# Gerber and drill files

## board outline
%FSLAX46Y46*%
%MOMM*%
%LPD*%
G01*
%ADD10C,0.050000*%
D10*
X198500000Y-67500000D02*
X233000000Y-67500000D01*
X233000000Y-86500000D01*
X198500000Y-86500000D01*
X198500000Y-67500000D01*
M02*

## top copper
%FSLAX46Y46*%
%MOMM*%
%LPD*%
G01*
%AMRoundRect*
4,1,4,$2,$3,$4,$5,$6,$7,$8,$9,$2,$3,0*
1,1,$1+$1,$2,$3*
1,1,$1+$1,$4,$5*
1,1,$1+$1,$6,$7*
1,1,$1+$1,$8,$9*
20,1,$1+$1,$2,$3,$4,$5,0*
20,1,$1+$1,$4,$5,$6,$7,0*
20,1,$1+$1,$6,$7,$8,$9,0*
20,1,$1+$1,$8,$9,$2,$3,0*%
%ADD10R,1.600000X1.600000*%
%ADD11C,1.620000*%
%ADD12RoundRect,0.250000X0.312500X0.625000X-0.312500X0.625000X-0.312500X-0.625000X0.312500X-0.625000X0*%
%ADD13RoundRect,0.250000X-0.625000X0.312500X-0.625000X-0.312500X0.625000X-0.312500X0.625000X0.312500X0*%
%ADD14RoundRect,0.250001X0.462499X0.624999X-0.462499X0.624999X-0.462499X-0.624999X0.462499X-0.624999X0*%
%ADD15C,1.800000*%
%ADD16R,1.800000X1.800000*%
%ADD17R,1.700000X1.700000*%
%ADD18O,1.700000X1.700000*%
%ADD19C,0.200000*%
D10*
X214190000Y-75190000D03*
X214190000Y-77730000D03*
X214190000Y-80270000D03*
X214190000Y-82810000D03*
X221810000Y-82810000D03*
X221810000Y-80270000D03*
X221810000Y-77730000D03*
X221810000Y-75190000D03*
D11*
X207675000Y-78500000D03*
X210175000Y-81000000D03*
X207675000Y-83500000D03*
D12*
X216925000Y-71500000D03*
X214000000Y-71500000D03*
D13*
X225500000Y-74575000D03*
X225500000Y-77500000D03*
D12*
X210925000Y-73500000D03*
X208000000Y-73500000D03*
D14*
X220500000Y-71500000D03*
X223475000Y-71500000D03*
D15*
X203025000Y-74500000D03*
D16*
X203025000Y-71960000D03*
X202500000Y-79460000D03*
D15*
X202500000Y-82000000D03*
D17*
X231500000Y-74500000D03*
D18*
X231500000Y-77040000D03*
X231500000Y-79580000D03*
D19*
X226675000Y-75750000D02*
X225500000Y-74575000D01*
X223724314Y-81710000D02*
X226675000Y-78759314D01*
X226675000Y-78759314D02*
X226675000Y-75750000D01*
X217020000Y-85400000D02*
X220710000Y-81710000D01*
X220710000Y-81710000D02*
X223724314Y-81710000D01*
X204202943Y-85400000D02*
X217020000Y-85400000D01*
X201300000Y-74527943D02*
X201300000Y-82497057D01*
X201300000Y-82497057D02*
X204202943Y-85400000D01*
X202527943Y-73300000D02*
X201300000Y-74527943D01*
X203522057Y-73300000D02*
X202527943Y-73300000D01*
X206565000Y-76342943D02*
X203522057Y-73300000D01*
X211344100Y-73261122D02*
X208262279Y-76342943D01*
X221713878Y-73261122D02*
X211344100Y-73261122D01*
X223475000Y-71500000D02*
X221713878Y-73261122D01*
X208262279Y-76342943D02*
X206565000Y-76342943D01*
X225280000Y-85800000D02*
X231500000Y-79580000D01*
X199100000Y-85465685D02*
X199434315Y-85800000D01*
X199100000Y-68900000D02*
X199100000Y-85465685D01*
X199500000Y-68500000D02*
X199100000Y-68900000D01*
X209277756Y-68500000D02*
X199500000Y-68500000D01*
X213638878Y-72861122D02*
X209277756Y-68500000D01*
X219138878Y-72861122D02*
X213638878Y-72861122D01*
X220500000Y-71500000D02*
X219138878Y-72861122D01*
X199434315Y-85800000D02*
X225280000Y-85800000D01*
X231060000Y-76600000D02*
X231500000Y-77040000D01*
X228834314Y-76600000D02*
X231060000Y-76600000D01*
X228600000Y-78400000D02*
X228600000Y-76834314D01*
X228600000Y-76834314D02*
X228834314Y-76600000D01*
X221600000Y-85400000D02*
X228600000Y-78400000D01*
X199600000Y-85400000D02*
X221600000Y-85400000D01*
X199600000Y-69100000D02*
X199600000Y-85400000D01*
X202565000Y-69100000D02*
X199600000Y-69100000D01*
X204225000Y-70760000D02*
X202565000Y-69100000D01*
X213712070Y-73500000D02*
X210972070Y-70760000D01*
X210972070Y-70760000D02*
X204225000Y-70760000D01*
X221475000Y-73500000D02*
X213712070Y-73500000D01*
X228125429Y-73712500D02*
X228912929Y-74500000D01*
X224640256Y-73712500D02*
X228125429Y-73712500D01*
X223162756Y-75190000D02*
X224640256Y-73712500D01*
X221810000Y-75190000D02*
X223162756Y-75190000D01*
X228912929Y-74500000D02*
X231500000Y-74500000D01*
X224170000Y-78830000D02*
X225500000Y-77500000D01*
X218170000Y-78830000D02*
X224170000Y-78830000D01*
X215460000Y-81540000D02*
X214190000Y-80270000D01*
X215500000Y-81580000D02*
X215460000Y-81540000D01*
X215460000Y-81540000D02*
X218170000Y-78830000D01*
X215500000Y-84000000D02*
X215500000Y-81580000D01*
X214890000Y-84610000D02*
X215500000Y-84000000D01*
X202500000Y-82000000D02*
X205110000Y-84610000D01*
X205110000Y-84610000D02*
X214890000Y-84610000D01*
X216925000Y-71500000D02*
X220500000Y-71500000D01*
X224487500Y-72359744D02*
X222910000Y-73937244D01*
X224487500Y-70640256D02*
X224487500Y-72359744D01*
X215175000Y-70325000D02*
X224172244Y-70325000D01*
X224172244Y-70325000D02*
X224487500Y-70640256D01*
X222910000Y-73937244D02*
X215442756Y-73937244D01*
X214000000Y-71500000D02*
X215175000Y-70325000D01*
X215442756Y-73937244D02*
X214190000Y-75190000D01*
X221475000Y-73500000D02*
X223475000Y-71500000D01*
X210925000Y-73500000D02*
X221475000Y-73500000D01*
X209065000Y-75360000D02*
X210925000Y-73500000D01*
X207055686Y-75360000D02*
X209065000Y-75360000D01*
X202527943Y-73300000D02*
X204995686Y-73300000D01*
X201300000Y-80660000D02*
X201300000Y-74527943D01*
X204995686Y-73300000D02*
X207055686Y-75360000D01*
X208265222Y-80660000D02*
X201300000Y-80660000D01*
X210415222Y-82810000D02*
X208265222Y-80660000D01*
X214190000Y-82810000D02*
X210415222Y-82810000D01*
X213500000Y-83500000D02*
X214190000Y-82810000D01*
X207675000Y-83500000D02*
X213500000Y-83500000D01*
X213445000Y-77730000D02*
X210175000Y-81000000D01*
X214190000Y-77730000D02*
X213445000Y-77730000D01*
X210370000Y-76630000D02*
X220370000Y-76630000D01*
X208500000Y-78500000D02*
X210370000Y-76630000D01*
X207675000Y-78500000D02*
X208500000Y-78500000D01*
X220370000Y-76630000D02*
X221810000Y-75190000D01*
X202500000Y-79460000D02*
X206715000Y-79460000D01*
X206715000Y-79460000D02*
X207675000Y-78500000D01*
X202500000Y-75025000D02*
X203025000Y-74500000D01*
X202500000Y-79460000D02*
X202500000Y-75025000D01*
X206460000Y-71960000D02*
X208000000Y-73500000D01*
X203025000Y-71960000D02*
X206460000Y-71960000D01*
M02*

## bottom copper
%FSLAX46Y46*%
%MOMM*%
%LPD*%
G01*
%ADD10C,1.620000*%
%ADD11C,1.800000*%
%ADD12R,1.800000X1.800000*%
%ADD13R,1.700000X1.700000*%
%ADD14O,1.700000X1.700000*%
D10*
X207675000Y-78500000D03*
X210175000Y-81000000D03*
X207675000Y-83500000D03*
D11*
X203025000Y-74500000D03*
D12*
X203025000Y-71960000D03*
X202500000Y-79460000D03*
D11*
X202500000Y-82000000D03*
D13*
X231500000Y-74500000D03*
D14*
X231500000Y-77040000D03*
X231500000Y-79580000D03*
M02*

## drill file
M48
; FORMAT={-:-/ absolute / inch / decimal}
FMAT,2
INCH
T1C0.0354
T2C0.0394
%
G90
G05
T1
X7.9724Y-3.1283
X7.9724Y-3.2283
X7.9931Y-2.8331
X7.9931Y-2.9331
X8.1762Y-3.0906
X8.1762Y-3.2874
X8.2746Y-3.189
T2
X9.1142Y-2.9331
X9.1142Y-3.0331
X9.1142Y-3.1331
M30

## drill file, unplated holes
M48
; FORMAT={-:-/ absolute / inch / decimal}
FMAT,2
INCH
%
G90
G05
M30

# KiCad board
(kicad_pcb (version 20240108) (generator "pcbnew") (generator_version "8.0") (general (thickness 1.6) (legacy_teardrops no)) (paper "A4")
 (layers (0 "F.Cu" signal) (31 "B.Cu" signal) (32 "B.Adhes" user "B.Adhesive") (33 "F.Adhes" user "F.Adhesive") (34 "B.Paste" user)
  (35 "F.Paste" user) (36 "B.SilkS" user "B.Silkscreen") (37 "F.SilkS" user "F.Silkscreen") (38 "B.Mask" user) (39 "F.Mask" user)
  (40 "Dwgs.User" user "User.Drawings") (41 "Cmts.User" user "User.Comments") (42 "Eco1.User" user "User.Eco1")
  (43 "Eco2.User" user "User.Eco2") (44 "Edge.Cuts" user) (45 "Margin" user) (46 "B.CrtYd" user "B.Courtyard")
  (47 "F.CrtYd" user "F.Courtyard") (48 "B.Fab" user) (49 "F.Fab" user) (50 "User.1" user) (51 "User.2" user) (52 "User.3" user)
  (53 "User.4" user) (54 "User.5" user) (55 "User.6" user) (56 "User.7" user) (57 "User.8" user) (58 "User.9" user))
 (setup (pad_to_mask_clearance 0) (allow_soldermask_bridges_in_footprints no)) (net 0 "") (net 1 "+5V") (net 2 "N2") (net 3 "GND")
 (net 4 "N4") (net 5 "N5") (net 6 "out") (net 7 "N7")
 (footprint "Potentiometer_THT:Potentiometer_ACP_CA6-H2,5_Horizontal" (layer "F.Cu") (at 207.675 78.5)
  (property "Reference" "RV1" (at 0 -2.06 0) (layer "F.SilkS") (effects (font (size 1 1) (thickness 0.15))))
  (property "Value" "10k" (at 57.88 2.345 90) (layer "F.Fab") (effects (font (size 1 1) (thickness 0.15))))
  (pad "1" thru_hole circle (at 0 0) (size 1.62 1.62) (drill 0.9) (layers "*.Cu" "*.Mask") (remove_unused_layers no) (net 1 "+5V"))
  (pad "2" thru_hole circle (at 2.5 2.5) (size 1.62 1.62) (drill 0.9) (layers "*.Cu" "*.Mask") (remove_unused_layers no) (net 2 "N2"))
  (pad "3" thru_hole circle (at 0 5) (size 1.62 1.62) (drill 0.9) (layers "*.Cu" "*.Mask") (remove_unused_layers no) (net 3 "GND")))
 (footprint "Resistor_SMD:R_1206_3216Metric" (layer "F.Cu") (at 209.4625 73.5 180)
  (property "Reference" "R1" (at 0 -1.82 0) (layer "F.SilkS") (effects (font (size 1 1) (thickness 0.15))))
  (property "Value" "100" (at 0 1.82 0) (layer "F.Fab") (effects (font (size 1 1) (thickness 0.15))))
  (pad "1" smd roundrect (at -1.4625 0 180) (size 1.125 1.75) (layers "F.Cu" "F.Paste" "F.Mask") (roundrect_rratio 0.222222) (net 3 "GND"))
  (pad "2" smd roundrect (at 1.4625 0 180) (size 1.125 1.75) (layers "F.Cu" "F.Paste" "F.Mask") (roundrect_rratio 0.222222) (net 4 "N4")))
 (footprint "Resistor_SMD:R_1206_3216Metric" (layer "F.Cu") (at 225.5 76.0375 -90)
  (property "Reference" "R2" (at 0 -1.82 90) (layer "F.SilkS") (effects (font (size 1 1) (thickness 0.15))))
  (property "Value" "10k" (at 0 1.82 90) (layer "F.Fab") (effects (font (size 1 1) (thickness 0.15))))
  (pad "1" smd roundrect (at -1.4625 0 270) (size 1.125 1.75) (layers "F.Cu" "F.Paste" "F.Mask") (roundrect_rratio 0.222222) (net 3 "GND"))
  (pad "2" smd roundrect (at 1.4625 0 270) (size 1.125 1.75) (layers "F.Cu" "F.Paste" "F.Mask") (roundrect_rratio 0.222222) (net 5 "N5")))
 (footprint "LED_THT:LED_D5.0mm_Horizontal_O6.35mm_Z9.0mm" (layer "F.Cu") (at 202.5 79.46 -90)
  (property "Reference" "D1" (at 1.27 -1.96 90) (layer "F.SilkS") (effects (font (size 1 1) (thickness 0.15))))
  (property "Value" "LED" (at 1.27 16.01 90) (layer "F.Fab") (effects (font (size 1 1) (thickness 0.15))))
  (pad "1" thru_hole rect (at 0 0 270) (size 1.8 1.8) (drill 0.9) (layers "*.Cu" "*.Mask") (remove_unused_layers no) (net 1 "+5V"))
  (pad "2" thru_hole circle (at 2.54 0 270) (size 1.8 1.8) (drill 0.9) (layers "*.Cu" "*.Mask") (remove_unused_layers no) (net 5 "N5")))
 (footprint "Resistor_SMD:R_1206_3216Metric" (layer "F.Cu") (at 215.4625 71.5 180)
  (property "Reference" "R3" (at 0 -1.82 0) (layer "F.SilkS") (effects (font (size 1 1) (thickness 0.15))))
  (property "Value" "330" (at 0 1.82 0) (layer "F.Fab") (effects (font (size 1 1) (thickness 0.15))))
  (pad "1" smd roundrect (at -1.4625 0 180) (size 1.125 1.75) (layers "F.Cu" "F.Paste" "F.Mask") (roundrect_rratio 0.222222) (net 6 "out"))
  (pad "2" smd roundrect (at 1.4625 0 180) (size 1.125 1.75) (layers "F.Cu" "F.Paste" "F.Mask") (roundrect_rratio 0.222222) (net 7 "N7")))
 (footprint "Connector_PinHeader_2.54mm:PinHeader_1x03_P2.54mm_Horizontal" (layer "F.Cu") (at 231.5 74.5)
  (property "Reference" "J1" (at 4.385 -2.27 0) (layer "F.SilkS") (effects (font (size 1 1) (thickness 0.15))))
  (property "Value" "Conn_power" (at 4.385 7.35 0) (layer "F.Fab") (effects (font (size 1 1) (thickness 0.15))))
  (pad "1" thru_hole rect (at 0 0) (size 1.7 1.7) (drill 1) (layers "*.Cu" "*.Mask") (remove_unused_layers no) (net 1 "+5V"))
  (pad "2" thru_hole oval (at 0 2.54) (size 1.7 1.7) (drill 1) (layers "*.Cu" "*.Mask") (remove_unused_layers no) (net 3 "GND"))
  (pad "3" thru_hole oval (at 0 5.08) (size 1.7 1.7) (drill 1) (layers "*.Cu" "*.Mask") (remove_unused_layers no) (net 6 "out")))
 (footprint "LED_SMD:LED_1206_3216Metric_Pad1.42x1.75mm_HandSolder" (layer "F.Cu") (at 221.9875 71.5 180)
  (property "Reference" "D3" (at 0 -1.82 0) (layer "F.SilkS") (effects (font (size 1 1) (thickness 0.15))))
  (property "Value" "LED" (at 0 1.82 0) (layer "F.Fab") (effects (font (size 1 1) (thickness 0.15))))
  (pad "1" smd roundrect (at -1.4875 0 180) (size 1.425 1.75) (layers "F.Cu" "F.Paste" "F.Mask") (roundrect_rratio 0.175439) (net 3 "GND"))
  (pad "2" smd roundrect (at 1.4875 0 180) (size 1.425 1.75) (layers "F.Cu" "F.Paste" "F.Mask") (roundrect_rratio 0.175439) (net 6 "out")))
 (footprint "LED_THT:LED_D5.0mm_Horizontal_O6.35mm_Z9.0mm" (layer "F.Cu") (at 203.025 71.96 -90)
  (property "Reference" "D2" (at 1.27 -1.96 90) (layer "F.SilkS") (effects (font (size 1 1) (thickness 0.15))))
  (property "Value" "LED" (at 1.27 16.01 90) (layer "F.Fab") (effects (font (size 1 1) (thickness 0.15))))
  (pad "1" thru_hole rect (at 0 0 270) (size 1.8 1.8) (drill 0.9) (layers "*.Cu" "*.Mask") (remove_unused_layers no) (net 4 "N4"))
  (pad "2" thru_hole circle (at 2.54 0 270) (size 1.8 1.8) (drill 0.9) (layers "*.Cu" "*.Mask") (remove_unused_layers no) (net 1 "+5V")))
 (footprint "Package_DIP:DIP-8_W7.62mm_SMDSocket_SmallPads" (layer "F.Cu") (at 218 79)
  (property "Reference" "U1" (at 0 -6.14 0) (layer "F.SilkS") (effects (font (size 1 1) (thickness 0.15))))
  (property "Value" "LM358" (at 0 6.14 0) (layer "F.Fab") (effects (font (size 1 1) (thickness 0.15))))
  (pad "1" smd rect (at -3.81 -3.81) (size 1.6 1.6) (layers "F.Cu" "F.Paste" "F.Mask") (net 7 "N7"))
  (pad "2" smd rect (at -3.81 -1.27) (size 1.6 1.6) (layers "F.Cu" "F.Paste" "F.Mask") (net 2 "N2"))
  (pad "3" smd rect (at -3.81 1.27) (size 1.6 1.6) (layers "F.Cu" "F.Paste" "F.Mask") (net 5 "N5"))
  (pad "4" smd rect (at -3.81 3.81) (size 1.6 1.6) (layers "F.Cu" "F.Paste" "F.Mask") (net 3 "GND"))
  (pad "5" smd rect (at 3.81 3.81) (size 1.6 1.6) (layers "F.Cu" "F.Paste" "F.Mask"))
  (pad "6" smd rect (at 3.81 1.27) (size 1.6 1.6) (layers "F.Cu" "F.Paste" "F.Mask"))
  (pad "7" smd rect (at 3.81 -1.27) (size 1.6 1.6) (layers "F.Cu" "F.Paste" "F.Mask"))
  (pad "8" smd rect (at 3.81 -3.81) (size 1.6 1.6) (layers "F.Cu" "F.Paste" "F.Mask") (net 1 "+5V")))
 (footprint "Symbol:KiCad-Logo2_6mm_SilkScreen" (layer "B.Cu") (at 224.5 70.5 180)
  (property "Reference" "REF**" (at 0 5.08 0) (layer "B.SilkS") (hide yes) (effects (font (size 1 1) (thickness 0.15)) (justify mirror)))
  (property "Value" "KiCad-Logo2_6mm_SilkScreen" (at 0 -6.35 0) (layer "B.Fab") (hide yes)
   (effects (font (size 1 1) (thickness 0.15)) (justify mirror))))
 (gr_rect (start 198.5 67.5) (end 233 86.5) (stroke (width 0.05) (type default)) (fill none) (layer "Edge.Cuts"))
 (segment (start 228.125429 73.7125) (end 228.912929 74.5) (width 0.2) (layer "F.Cu") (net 1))
 (segment (start 208.5 78.5) (end 210.37 76.63) (width 0.2) (layer "F.Cu") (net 1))
 (segment (start 224.640256 73.7125) (end 228.125429 73.7125) (width 0.2) (layer "F.Cu") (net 1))
 (segment (start 220.37 76.63) (end 221.81 75.19) (width 0.2) (layer "F.Cu") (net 1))
 (segment (start 223.162756 75.19) (end 224.640256 73.7125) (width 0.2) (layer "F.Cu") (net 1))
 (segment (start 210.37 76.63) (end 220.37 76.63) (width 0.2) (layer "F.Cu") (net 1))
 (segment (start 206.715 79.46) (end 207.675 78.5) (width 0.2) (layer "F.Cu") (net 1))
 (segment (start 221.81 75.19) (end 223.162756 75.19) (width 0.2) (layer "F.Cu") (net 1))
 (segment (start 202.5 79.46) (end 206.715 79.46) (width 0.2) (layer "F.Cu") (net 1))
 (segment (start 228.912929 74.5) (end 231.5 74.5) (width 0.2) (layer "F.Cu") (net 1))
 (segment (start 202.5 75.025) (end 203.025 74.5) (width 0.2) (layer "F.Cu") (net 1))
 (segment (start 207.675 78.5) (end 208.5 78.5) (width 0.2) (layer "F.Cu") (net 1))
 (segment (start 202.5 79.46) (end 202.5 75.025) (width 0.2) (layer "F.Cu") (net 1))
 (segment (start 224.17 78.83) (end 225.5 77.5) (width 0.2) (layer "F.Cu") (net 5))
 (segment (start 214.89 84.61) (end 215.5 84) (width 0.2) (layer "F.Cu") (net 5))
 (segment (start 205.11 84.61) (end 214.89 84.61) (width 0.2) (layer "F.Cu") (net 5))
 (segment (start 202.5 82) (end 205.11 84.61) (width 0.2) (layer "F.Cu") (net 5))
 (segment (start 218.17 78.83) (end 224.17 78.83) (width 0.2) (layer "F.Cu") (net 5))
 (segment (start 215.5 81.58) (end 215.46 81.54) (width 0.2) (layer "F.Cu") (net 5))
 (segment (start 215.46 81.54) (end 218.17 78.83) (width 0.2) (layer "F.Cu") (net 5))
 (segment (start 215.46 81.54) (end 214.19 80.27) (width 0.2) (layer "F.Cu") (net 5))
 (segment (start 215.5 84) (end 215.5 81.58) (width 0.2) (layer "F.Cu") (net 5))
 (segment (start 203.025 71.96) (end 206.46 71.96) (width 0.2) (layer "F.Cu") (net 4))
 (segment (start 206.46 71.96) (end 208 73.5) (width 0.2) (layer "F.Cu") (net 4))
 (segment (start 226.675 75.75) (end 225.5 74.575) (width 0.2) (layer "F.Cu") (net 3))
 (segment (start 201.3 80.66) (end 201.3 74.527943) (width 0.2) (layer "F.Cu") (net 3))
 (segment (start 228.6 76.834314) (end 228.834314 76.6) (width 0.2) (layer "F.Cu") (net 3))
 (segment (start 208.265222 80.66) (end 201.3 80.66) (width 0.2) (layer "F.Cu") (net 3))
 (segment (start 223.724314 81.71) (end 226.675 78.759314) (width 0.2) (layer "F.Cu") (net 3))
 (segment (start 199.6 85.4) (end 221.6 85.4) (width 0.2) (layer "F.Cu") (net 3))
 (segment (start 208.262279 76.342943) (end 206.565 76.342943) (width 0.2) (layer "F.Cu") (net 3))
 (segment (start 202.565 69.1) (end 199.6 69.1) (width 0.2) (layer "F.Cu") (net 3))
 (segment (start 231.06 76.6) (end 231.5 77.04) (width 0.2) (layer "F.Cu") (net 3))
 (segment (start 204.225 70.76) (end 202.565 69.1) (width 0.2) (layer "F.Cu") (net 3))
 (segment (start 207.675 83.5) (end 213.5 83.5) (width 0.2) (layer "F.Cu") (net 3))
 (segment (start 207.055686 75.36) (end 209.065 75.36) (width 0.2) (layer "F.Cu") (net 3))
 (segment (start 209.065 75.36) (end 210.925 73.5) (width 0.2) (layer "F.Cu") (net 3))
 (segment (start 202.527943 73.3) (end 204.995686 73.3) (width 0.2) (layer "F.Cu") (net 3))
 (segment (start 206.565 76.342943) (end 203.522057 73.3) (width 0.2) (layer "F.Cu") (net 3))
 (segment (start 202.527943 73.3) (end 201.3 74.527943) (width 0.2) (layer "F.Cu") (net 3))
 (segment (start 223.475 71.5) (end 221.713878 73.261122) (width 0.2) (layer "F.Cu") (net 3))
 (segment (start 214.19 82.81) (end 210.415222 82.81) (width 0.2) (layer "F.Cu") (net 3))
 (segment (start 217.02 85.4) (end 220.71 81.71) (width 0.2) (layer "F.Cu") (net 3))
 (segment (start 203.522057 73.3) (end 202.527943 73.3) (width 0.2) (layer "F.Cu") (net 3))
 (segment (start 226.675 78.759314) (end 226.675 75.75) (width 0.2) (layer "F.Cu") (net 3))
 (segment (start 210.97207 70.76) (end 204.225 70.76) (width 0.2) (layer "F.Cu") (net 3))
 (segment (start 220.71 81.71) (end 223.724314 81.71) (width 0.2) (layer "F.Cu") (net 3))
 (segment (start 221.6 85.4) (end 228.6 78.4) (width 0.2) (layer "F.Cu") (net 3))
 (segment (start 204.995686 73.3) (end 207.055686 75.36) (width 0.2) (layer "F.Cu") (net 3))
 (segment (start 228.834314 76.6) (end 231.06 76.6) (width 0.2) (layer "F.Cu") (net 3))
 (segment (start 210.925 73.5) (end 221.475 73.5) (width 0.2) (layer "F.Cu") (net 3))
 (segment (start 211.3441 73.261122) (end 208.262279 76.342943) (width 0.2) (layer "F.Cu") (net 3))
 (segment (start 221.475 73.5) (end 213.71207 73.5) (width 0.2) (layer "F.Cu") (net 3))
 (segment (start 201.3 74.527943) (end 201.3 82.497057) (width 0.2) (layer "F.Cu") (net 3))
 (segment (start 228.6 78.4) (end 228.6 76.834314) (width 0.2) (layer "F.Cu") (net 3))
 (segment (start 210.415222 82.81) (end 208.265222 80.66) (width 0.2) (layer "F.Cu") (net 3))
 (segment (start 204.202943 85.4) (end 217.02 85.4) (width 0.2) (layer "F.Cu") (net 3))
 (segment (start 213.5 83.5) (end 214.19 82.81) (width 0.2) (layer "F.Cu") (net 3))
 (segment (start 221.475 73.5) (end 223.475 71.5) (width 0.2) (layer "F.Cu") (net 3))
 (segment (start 201.3 82.497057) (end 204.202943 85.4) (width 0.2) (layer "F.Cu") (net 3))
 (segment (start 213.71207 73.5) (end 210.97207 70.76) (width 0.2) (layer "F.Cu") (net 3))
 (segment (start 199.6 69.1) (end 199.6 85.4) (width 0.2) (layer "F.Cu") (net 3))
 (segment (start 221.713878 73.261122) (end 211.3441 73.261122) (width 0.2) (layer "F.Cu") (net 3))
 (segment (start 225.28 85.8) (end 231.5 79.58) (width 0.2) (layer "F.Cu") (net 6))
 (segment (start 199.1 85.465685) (end 199.434315 85.8) (width 0.2) (layer "F.Cu") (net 6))
 (segment (start 216.925 71.5) (end 220.5 71.5) (width 0.2) (layer "F.Cu") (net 6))
 (segment (start 199.434315 85.8) (end 225.28 85.8) (width 0.2) (layer "F.Cu") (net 6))
 (segment (start 213.638878 72.861122) (end 209.277756 68.5) (width 0.2) (layer "F.Cu") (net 6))
 (segment (start 199.1 68.9) (end 199.1 85.465685) (width 0.2) (layer "F.Cu") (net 6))
 (segment (start 220.5 71.5) (end 219.138878 72.861122) (width 0.2) (layer "F.Cu") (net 6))
 (segment (start 199.5 68.5) (end 199.1 68.9) (width 0.2) (layer "F.Cu") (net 6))
 (segment (start 209.277756 68.5) (end 199.5 68.5) (width 0.2) (layer "F.Cu") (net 6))
 (segment (start 219.138878 72.861122) (end 213.638878 72.861122) (width 0.2) (layer "F.Cu") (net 6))
 (segment (start 214 71.5) (end 215.175 70.325) (width 0.2) (layer "F.Cu") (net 7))
 (segment (start 215.442756 73.937244) (end 214.19 75.19) (width 0.2) (layer "F.Cu") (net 7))
 (segment (start 222.91 73.937244) (end 215.442756 73.937244) (width 0.2) (layer "F.Cu") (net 7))
 (segment (start 215.175 70.325) (end 224.172244 70.325) (width 0.2) (layer "F.Cu") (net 7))
 (segment (start 224.172244 70.325) (end 224.4875 70.640256) (width 0.2) (layer "F.Cu") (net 7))
 (segment (start 224.4875 72.359744) (end 222.91 73.937244) (width 0.2) (layer "F.Cu") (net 7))
 (segment (start 224.4875 70.640256) (end 224.4875 72.359744) (width 0.2) (layer "F.Cu") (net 7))
 (segment (start 213.445 77.73) (end 210.175 81) (width 0.2) (layer "F.Cu") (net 2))
 (segment (start 214.19 77.73) (end 213.445 77.73) (width 0.2) (layer "F.Cu") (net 2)))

